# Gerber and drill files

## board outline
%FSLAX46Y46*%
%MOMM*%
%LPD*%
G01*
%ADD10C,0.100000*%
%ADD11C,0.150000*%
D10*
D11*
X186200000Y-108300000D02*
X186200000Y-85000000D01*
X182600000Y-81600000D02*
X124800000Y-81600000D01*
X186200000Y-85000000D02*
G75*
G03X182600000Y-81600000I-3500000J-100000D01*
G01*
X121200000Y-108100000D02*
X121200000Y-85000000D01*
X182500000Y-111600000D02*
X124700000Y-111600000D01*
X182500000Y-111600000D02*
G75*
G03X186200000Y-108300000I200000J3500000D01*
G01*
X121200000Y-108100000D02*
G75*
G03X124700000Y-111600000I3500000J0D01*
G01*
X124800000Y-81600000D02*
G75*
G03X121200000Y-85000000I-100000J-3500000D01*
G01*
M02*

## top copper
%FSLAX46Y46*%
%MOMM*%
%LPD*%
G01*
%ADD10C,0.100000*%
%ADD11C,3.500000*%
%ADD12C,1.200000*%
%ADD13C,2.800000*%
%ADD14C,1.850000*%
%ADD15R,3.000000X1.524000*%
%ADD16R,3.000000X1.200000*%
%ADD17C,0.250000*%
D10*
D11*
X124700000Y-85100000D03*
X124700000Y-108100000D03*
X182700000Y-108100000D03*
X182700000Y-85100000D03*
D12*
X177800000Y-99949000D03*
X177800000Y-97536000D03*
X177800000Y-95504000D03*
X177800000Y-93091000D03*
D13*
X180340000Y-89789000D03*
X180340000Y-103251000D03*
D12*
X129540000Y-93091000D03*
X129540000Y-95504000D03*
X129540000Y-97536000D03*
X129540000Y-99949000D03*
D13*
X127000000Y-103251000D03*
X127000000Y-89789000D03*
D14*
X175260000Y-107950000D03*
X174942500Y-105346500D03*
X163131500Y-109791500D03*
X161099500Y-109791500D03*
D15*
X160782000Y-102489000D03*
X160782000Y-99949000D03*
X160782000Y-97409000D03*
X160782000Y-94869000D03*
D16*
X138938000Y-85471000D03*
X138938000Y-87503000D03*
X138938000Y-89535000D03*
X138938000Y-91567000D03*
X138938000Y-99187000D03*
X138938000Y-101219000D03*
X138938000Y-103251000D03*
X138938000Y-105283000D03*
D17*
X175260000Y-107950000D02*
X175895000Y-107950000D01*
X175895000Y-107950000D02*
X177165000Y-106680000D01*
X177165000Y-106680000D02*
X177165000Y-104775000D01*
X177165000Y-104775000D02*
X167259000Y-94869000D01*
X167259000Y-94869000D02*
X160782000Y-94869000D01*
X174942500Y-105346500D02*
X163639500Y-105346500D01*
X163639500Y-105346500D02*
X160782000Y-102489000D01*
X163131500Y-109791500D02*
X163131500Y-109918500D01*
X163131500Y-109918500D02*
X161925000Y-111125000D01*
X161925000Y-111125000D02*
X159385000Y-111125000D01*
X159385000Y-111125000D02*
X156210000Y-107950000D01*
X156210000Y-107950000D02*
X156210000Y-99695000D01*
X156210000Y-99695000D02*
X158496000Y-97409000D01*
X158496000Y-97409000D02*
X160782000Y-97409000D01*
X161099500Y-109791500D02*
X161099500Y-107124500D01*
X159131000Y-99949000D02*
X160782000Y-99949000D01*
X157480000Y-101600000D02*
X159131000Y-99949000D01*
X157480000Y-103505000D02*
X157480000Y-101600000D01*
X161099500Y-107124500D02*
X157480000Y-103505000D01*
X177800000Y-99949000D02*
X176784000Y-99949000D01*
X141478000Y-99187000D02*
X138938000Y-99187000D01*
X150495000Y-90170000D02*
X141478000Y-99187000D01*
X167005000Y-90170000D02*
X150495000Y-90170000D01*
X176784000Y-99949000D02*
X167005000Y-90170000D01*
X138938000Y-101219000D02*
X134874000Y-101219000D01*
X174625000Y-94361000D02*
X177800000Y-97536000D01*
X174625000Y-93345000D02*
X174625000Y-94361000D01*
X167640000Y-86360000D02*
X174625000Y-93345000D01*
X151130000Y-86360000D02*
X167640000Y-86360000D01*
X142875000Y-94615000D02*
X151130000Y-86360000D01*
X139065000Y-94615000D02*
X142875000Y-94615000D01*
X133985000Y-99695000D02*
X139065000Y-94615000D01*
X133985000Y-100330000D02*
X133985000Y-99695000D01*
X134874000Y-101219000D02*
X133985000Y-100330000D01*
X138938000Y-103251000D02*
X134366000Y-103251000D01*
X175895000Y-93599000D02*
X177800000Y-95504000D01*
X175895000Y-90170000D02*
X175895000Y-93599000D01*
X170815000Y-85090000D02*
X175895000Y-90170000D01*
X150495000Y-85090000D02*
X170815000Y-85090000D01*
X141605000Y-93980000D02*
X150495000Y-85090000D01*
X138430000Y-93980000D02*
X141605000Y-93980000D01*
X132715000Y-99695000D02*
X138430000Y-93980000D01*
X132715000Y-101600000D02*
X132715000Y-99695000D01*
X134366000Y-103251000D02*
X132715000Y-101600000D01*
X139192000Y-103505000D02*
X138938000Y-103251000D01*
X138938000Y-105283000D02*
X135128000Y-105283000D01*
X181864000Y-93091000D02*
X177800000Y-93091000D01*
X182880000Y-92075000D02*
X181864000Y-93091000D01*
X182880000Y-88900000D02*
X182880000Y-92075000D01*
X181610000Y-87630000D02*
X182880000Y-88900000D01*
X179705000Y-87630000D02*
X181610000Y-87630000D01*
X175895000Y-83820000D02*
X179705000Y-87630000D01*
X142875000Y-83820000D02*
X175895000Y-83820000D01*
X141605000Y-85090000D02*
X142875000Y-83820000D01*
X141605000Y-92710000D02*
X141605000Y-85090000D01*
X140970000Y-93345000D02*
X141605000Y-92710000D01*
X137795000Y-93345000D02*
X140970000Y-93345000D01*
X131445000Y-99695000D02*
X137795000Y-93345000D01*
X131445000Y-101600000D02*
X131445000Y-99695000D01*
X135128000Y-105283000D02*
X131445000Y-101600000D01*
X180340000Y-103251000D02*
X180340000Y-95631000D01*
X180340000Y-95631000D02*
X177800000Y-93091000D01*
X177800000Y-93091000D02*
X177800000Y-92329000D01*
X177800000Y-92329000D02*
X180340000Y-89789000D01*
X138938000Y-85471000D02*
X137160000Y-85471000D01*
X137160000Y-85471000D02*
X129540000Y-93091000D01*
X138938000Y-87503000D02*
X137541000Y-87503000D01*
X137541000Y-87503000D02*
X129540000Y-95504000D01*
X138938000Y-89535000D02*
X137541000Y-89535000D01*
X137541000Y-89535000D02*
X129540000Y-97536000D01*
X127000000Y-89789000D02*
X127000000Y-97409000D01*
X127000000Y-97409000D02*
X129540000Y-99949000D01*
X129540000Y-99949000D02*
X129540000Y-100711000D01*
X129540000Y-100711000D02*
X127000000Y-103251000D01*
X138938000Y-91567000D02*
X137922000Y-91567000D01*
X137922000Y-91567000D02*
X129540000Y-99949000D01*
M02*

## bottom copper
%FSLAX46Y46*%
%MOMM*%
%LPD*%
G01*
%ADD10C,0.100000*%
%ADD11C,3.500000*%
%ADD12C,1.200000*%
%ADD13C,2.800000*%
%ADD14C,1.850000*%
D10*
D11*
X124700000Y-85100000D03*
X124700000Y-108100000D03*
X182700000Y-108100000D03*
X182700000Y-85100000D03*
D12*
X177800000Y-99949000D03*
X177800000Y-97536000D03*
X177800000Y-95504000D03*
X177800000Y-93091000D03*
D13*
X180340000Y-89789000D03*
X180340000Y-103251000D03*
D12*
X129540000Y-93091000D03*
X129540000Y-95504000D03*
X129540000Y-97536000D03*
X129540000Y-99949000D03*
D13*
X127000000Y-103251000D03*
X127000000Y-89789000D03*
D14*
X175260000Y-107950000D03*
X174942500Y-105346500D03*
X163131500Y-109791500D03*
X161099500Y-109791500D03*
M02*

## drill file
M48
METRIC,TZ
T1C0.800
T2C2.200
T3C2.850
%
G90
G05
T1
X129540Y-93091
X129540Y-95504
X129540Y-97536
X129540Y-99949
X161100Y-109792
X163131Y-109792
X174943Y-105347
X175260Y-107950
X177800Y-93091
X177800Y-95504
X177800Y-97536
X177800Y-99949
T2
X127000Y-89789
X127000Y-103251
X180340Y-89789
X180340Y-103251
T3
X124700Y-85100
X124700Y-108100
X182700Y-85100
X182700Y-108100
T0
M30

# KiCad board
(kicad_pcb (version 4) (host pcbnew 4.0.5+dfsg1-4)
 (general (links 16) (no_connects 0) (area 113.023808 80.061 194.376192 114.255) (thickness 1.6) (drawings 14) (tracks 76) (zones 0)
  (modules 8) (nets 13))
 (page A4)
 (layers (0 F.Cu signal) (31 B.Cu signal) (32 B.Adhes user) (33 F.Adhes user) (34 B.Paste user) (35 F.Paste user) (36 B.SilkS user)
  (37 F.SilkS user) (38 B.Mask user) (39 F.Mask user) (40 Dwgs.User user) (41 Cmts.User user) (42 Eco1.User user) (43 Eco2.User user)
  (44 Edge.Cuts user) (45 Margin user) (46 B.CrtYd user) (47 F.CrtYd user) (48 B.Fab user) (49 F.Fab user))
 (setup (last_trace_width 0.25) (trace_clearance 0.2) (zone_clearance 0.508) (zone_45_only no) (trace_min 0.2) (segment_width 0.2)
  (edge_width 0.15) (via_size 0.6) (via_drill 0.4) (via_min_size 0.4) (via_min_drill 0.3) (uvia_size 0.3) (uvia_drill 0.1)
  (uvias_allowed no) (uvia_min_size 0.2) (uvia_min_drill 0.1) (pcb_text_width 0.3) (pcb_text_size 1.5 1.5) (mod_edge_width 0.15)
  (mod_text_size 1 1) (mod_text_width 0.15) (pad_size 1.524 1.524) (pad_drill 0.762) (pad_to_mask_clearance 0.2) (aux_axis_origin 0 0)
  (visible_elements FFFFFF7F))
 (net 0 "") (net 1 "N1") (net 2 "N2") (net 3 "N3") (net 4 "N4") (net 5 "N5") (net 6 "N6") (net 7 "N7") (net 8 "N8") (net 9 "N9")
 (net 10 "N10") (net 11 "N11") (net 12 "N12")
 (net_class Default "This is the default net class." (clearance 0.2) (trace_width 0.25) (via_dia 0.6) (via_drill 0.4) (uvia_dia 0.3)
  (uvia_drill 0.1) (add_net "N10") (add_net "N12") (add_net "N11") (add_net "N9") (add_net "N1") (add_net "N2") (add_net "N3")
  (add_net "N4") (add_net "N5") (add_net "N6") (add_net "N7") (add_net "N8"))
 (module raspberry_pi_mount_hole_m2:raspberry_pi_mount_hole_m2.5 (layer F.Cu) (at 124.7 85.1)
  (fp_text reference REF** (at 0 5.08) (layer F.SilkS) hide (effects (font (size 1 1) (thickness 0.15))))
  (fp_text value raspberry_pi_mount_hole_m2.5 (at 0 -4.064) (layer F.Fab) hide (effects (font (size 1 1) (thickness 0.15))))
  (pad 1 thru_hole circle (at 0 0) (size 3.5 3.5) (drill 2.85) (layers *.Cu *.Mask)))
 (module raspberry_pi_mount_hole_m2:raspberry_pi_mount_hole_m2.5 (layer F.Cu) (at 124.7 108.1)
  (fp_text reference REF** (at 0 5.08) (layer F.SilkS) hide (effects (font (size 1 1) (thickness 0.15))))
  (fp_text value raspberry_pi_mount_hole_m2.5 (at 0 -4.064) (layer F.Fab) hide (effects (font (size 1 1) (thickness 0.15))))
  (pad 1 thru_hole circle (at 0 0) (size 3.5 3.5) (drill 2.85) (layers *.Cu *.Mask)))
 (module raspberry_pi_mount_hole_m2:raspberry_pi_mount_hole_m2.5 (layer F.Cu) (at 182.7 108.1)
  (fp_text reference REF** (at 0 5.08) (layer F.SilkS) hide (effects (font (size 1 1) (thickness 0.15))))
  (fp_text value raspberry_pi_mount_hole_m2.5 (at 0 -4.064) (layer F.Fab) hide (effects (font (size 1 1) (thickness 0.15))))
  (pad 1 thru_hole circle (at 0 0) (size 3.5 3.5) (drill 2.85) (layers *.Cu *.Mask)))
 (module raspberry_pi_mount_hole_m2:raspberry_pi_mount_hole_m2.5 (layer F.Cu) (at 182.7 85.1)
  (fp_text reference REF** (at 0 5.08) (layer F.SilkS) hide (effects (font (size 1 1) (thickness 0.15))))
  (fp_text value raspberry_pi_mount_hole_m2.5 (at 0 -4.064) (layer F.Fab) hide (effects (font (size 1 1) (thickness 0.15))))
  (pad 1 thru_hole circle (at 0 0) (size 3.5 3.5) (drill 2.85) (layers *.Cu *.Mask)))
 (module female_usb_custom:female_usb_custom (layer F.Cu) (at 177.8 96.52 90)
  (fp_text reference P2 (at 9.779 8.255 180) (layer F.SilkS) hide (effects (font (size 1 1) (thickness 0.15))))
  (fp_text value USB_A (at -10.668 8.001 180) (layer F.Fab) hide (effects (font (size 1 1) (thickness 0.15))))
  (pad 1 thru_hole circle (at -3.429 0 90) (size 1.2 1.2) (drill 0.8) (layers *.Cu *.Mask F.SilkS) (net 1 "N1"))
  (pad 2 thru_hole circle (at -1.016 0 90) (size 1.2 1.2) (drill 0.8) (layers *.Cu *.Mask F.SilkS) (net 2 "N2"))
  (pad 3 thru_hole circle (at 1.016 0 90) (size 1.2 1.2) (drill 0.8) (layers *.Cu *.Mask F.SilkS) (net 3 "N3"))
  (pad 4 thru_hole circle (at 3.429 0 90) (size 1.2 1.2) (drill 0.8) (layers *.Cu *.Mask F.SilkS) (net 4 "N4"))
  (pad 4 thru_hole circle (at 6.731 2.54 90) (size 2.8 2.8) (drill 2.2) (layers *.Cu *.Mask F.SilkS) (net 4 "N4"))
  (pad 4 thru_hole circle (at -6.731 2.54 90) (size 2.8 2.8) (drill 2.2) (layers *.Cu *.Mask F.SilkS) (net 4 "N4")))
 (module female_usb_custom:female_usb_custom (layer F.Cu) (at 129.54 96.52 270)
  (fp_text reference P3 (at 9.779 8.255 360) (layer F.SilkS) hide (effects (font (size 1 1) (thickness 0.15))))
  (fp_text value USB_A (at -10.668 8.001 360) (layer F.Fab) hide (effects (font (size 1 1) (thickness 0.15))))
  (pad 1 thru_hole circle (at -3.429 0 270) (size 1.2 1.2) (drill 0.8) (layers *.Cu *.Mask F.SilkS) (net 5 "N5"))
  (pad 2 thru_hole circle (at -1.016 0 270) (size 1.2 1.2) (drill 0.8) (layers *.Cu *.Mask F.SilkS) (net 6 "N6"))
  (pad 3 thru_hole circle (at 1.016 0 270) (size 1.2 1.2) (drill 0.8) (layers *.Cu *.Mask F.SilkS) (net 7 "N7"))
  (pad 4 thru_hole circle (at 3.429 0 270) (size 1.2 1.2) (drill 0.8) (layers *.Cu *.Mask F.SilkS) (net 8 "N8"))
  (pad 4 thru_hole circle (at 6.731 2.54 270) (size 2.8 2.8) (drill 2.2) (layers *.Cu *.Mask F.SilkS) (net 8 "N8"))
  (pad 4 thru_hole circle (at -6.731 2.54 270) (size 2.8 2.8) (drill 2.2) (layers *.Cu *.Mask F.SilkS) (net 8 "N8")))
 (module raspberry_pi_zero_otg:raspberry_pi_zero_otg (layer F.Cu) (at 175.26 107.95)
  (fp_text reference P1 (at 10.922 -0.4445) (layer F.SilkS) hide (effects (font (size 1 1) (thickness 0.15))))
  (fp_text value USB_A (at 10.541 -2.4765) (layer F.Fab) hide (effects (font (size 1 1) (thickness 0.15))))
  (pad 4 thru_hole circle (at 0 0) (size 1.85 1.85) (drill 0.8) (layers *.Cu *.Mask) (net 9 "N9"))
  (pad 1 thru_hole circle (at -0.3175 -2.6035) (size 1.85 1.85) (drill 0.8) (layers *.Cu *.Mask) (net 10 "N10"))
  (pad 3 thru_hole circle (at -12.1285 1.8415) (size 1.85 1.85) (drill 0.8) (layers *.Cu *.Mask) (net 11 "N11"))
  (pad 2 thru_hole circle (at -14.1605 1.8415) (size 1.85 1.85) (drill 0.8) (layers *.Cu *.Mask) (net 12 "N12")))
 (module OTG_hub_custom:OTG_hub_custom (layer F.Cu) (at 149.86 95.885 270)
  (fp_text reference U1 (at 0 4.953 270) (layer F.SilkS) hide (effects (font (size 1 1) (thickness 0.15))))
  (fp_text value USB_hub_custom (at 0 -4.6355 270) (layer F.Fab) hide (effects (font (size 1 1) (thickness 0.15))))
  (pad 1 smd rect (at 6.604 -10.922 270) (size 1.524 3) (layers F.Cu F.Paste F.Mask) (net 10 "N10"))
  (pad 2 smd rect (at 4.064 -10.922 270) (size 1.524 3) (layers F.Cu F.Paste F.Mask) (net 12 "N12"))
  (pad 3 smd rect (at 1.524 -10.922 270) (size 1.524 3) (layers F.Cu F.Paste F.Mask) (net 11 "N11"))
  (pad 4 smd rect (at -1.016 -10.922 270) (size 1.524 3) (layers F.Cu F.Paste F.Mask) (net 9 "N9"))
  (pad 5 smd rect (at -10.414 10.922 270) (size 1.2 3) (layers F.Cu F.Paste F.Mask) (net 5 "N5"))
  (pad 6 smd rect (at -8.382 10.922 270) (size 1.2 3) (layers F.Cu F.Paste F.Mask) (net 6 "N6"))
  (pad 7 smd rect (at -6.35 10.922 270) (size 1.2 3) (layers F.Cu F.Paste F.Mask) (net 7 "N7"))
  (pad 8 smd rect (at -4.318 10.922 270) (size 1.2 3) (layers F.Cu F.Paste F.Mask) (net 8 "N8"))
  (pad 9 smd rect (at 3.302 10.922 270) (size 1.2 3) (layers F.Cu F.Paste F.Mask) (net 1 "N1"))
  (pad 10 smd rect (at 5.334 10.922 270) (size 1.2 3) (layers F.Cu F.Paste F.Mask) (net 2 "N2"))
  (pad 11 smd rect (at 7.366 10.922 270) (size 1.2 3) (layers F.Cu F.Paste F.Mask) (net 3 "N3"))
  (pad 12 smd rect (at 9.398 10.922 270) (size 1.2 3) (layers F.Cu F.Paste F.Mask) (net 4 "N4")))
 (gr_line (start 186.2 108.3) (end 186.2 85) (angle 90) (layer Edge.Cuts) (width 0.15))
 (gr_line (start 182.6 81.6) (end 124.8 81.6) (angle 90) (layer Edge.Cuts) (width 0.15))
 (gr_arc (start 182.7 85.1) (end 182.6 81.6) (angle 90) (layer Edge.Cuts) (width 0.15))
 (gr_line (start 121.2 108.1) (end 121.2 85) (angle 90) (layer Edge.Cuts) (width 0.15))
 (gr_line (start 182.5 111.6) (end 124.7 111.6) (angle 90) (layer Edge.Cuts) (width 0.15))
 (gr_arc (start 182.7 108.1) (end 186.2 108.3) (angle 90) (layer Edge.Cuts) (width 0.15))
 (gr_arc (start 124.7 108.1) (end 124.7 111.6) (angle 90) (layer Edge.Cuts) (width 0.15))
 (gr_arc (start 124.7 85.1) (end 121.2 85) (angle 90) (layer Edge.Cuts) (width 0.15))
 (segment (start 175.26 107.95) (end 175.895 107.95) (width 0.25) (layer F.Cu) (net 9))
 (segment (start 175.895 107.95) (end 177.165 106.68) (width 0.25) (layer F.Cu) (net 9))
 (segment (start 177.165 106.68) (end 177.165 104.775) (width 0.25) (layer F.Cu) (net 9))
 (segment (start 177.165 104.775) (end 167.259 94.869) (width 0.25) (layer F.Cu) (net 9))
 (segment (start 167.259 94.869) (end 160.782 94.869) (width 0.25) (layer F.Cu) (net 9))
 (segment (start 174.9425 105.3465) (end 163.6395 105.3465) (width 0.25) (layer F.Cu) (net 10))
 (segment (start 163.6395 105.3465) (end 160.782 102.489) (width 0.25) (layer F.Cu) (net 10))
 (segment (start 163.1315 109.7915) (end 163.1315 109.9185) (width 0.25) (layer F.Cu) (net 11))
 (segment (start 163.1315 109.9185) (end 161.925 111.125) (width 0.25) (layer F.Cu) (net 11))
 (segment (start 161.925 111.125) (end 159.385 111.125) (width 0.25) (layer F.Cu) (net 11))
 (segment (start 159.385 111.125) (end 156.21 107.95) (width 0.25) (layer F.Cu) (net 11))
 (segment (start 156.21 107.95) (end 156.21 99.695) (width 0.25) (layer F.Cu) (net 11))
 (segment (start 156.21 99.695) (end 158.496 97.409) (width 0.25) (layer F.Cu) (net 11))
 (segment (start 158.496 97.409) (end 160.782 97.409) (width 0.25) (layer F.Cu) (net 11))
 (segment (start 161.0995 109.7915) (end 161.0995 107.1245) (width 0.25) (layer F.Cu) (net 12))
 (segment (start 159.131 99.949) (end 160.782 99.949) (width 0.25) (layer F.Cu) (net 12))
 (segment (start 157.48 101.6) (end 159.131 99.949) (width 0.25) (layer F.Cu) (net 12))
 (segment (start 157.48 103.505) (end 157.48 101.6) (width 0.25) (layer F.Cu) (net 12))
 (segment (start 161.0995 107.1245) (end 157.48 103.505) (width 0.25) (layer F.Cu) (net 12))
 (segment (start 177.8 99.949) (end 176.784 99.949) (width 0.25) (layer F.Cu) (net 1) (status 400000))
 (segment (start 141.478 99.187) (end 138.938 99.187) (width 0.25) (layer F.Cu) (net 1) (status 800000))
 (segment (start 150.495 90.17) (end 141.478 99.187) (width 0.25) (layer F.Cu) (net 1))
 (segment (start 167.005 90.17) (end 150.495 90.17) (width 0.25) (layer F.Cu) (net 1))
 (segment (start 176.784 99.949) (end 167.005 90.17) (width 0.25) (layer F.Cu) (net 1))
 (segment (start 138.938 101.219) (end 134.874 101.219) (width 0.25) (layer F.Cu) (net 2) (status 400000))
 (segment (start 174.625 94.361) (end 177.8 97.536) (width 0.25) (layer F.Cu) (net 2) (status 800000))
 (segment (start 174.625 93.345) (end 174.625 94.361) (width 0.25) (layer F.Cu) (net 2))
 (segment (start 167.64 86.36) (end 174.625 93.345) (width 0.25) (layer F.Cu) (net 2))
 (segment (start 151.13 86.36) (end 167.64 86.36) (width 0.25) (layer F.Cu) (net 2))
 (segment (start 142.875 94.615) (end 151.13 86.36) (width 0.25) (layer F.Cu) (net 2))
 (segment (start 139.065 94.615) (end 142.875 94.615) (width 0.25) (layer F.Cu) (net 2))
 (segment (start 133.985 99.695) (end 139.065 94.615) (width 0.25) (layer F.Cu) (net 2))
 (segment (start 133.985 100.33) (end 133.985 99.695) (width 0.25) (layer F.Cu) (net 2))
 (segment (start 134.874 101.219) (end 133.985 100.33) (width 0.25) (layer F.Cu) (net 2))
 (segment (start 138.938 103.251) (end 134.366 103.251) (width 0.25) (layer F.Cu) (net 3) (status 400000))
 (segment (start 175.895 93.599) (end 177.8 95.504) (width 0.25) (layer F.Cu) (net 3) (status 800000))
 (segment (start 175.895 90.17) (end 175.895 93.599) (width 0.25) (layer F.Cu) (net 3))
 (segment (start 170.815 85.09) (end 175.895 90.17) (width 0.25) (layer F.Cu) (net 3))
 (segment (start 150.495 85.09) (end 170.815 85.09) (width 0.25) (layer F.Cu) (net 3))
 (segment (start 141.605 93.98) (end 150.495 85.09) (width 0.25) (layer F.Cu) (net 3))
 (segment (start 138.43 93.98) (end 141.605 93.98) (width 0.25) (layer F.Cu) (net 3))
 (segment (start 132.715 99.695) (end 138.43 93.98) (width 0.25) (layer F.Cu) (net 3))
 (segment (start 132.715 101.6) (end 132.715 99.695) (width 0.25) (layer F.Cu) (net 3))
 (segment (start 134.366 103.251) (end 132.715 101.6) (width 0.25) (layer F.Cu) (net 3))
 (segment (start 139.192 103.505) (end 138.938 103.251) (width 0.25) (layer F.Cu) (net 3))
 (segment (start 138.938 105.283) (end 135.128 105.283) (width 0.25) (layer F.Cu) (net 4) (status 400000))
 (segment (start 181.864 93.091) (end 177.8 93.091) (width 0.25) (layer F.Cu) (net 4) (status 800000))
 (segment (start 182.88 92.075) (end 181.864 93.091) (width 0.25) (layer F.Cu) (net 4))
 (segment (start 182.88 88.9) (end 182.88 92.075) (width 0.25) (layer F.Cu) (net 4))
 (segment (start 181.61 87.63) (end 182.88 88.9) (width 0.25) (layer F.Cu) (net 4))
 (segment (start 179.705 87.63) (end 181.61 87.63) (width 0.25) (layer F.Cu) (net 4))
 (segment (start 175.895 83.82) (end 179.705 87.63) (width 0.25) (layer F.Cu) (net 4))
 (segment (start 142.875 83.82) (end 175.895 83.82) (width 0.25) (layer F.Cu) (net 4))
 (segment (start 141.605 85.09) (end 142.875 83.82) (width 0.25) (layer F.Cu) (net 4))
 (segment (start 141.605 92.71) (end 141.605 85.09) (width 0.25) (layer F.Cu) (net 4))
 (segment (start 140.97 93.345) (end 141.605 92.71) (width 0.25) (layer F.Cu) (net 4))
 (segment (start 137.795 93.345) (end 140.97 93.345) (width 0.25) (layer F.Cu) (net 4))
 (segment (start 131.445 99.695) (end 137.795 93.345) (width 0.25) (layer F.Cu) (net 4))
 (segment (start 131.445 101.6) (end 131.445 99.695) (width 0.25) (layer F.Cu) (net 4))
 (segment (start 135.128 105.283) (end 131.445 101.6) (width 0.25) (layer F.Cu) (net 4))
 (segment (start 180.34 103.251) (end 180.34 95.631) (width 0.25) (layer F.Cu) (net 4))
 (segment (start 180.34 95.631) (end 177.8 93.091) (width 0.25) (layer F.Cu) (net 4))
 (segment (start 177.8 93.091) (end 177.8 92.329) (width 0.25) (layer F.Cu) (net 4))
 (segment (start 177.8 92.329) (end 180.34 89.789) (width 0.25) (layer F.Cu) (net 4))
 (segment (start 138.938 85.471) (end 137.16 85.471) (width 0.25) (layer F.Cu) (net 5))
 (segment (start 137.16 85.471) (end 129.54 93.091) (width 0.25) (layer F.Cu) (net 5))
 (segment (start 138.938 87.503) (end 137.541 87.503) (width 0.25) (layer F.Cu) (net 6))
 (segment (start 137.541 87.503) (end 129.54 95.504) (width 0.25) (layer F.Cu) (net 6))
 (segment (start 138.938 89.535) (end 137.541 89.535) (width 0.25) (layer F.Cu) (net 7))
 (segment (start 137.541 89.535) (end 129.54 97.536) (width 0.25) (layer F.Cu) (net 7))
 (segment (start 127 89.789) (end 127 97.409) (width 0.25) (layer F.Cu) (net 8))
 (segment (start 127 97.409) (end 129.54 99.949) (width 0.25) (layer F.Cu) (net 8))
 (segment (start 129.54 99.949) (end 129.54 100.711) (width 0.25) (layer F.Cu) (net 8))
 (segment (start 129.54 100.711) (end 127 103.251) (width 0.25) (layer F.Cu) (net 8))
 (segment (start 138.938 91.567) (end 137.922 91.567) (width 0.25) (layer F.Cu) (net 8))
 (segment (start 137.922 91.567) (end 129.54 99.949) (width 0.25) (layer F.Cu) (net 8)))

